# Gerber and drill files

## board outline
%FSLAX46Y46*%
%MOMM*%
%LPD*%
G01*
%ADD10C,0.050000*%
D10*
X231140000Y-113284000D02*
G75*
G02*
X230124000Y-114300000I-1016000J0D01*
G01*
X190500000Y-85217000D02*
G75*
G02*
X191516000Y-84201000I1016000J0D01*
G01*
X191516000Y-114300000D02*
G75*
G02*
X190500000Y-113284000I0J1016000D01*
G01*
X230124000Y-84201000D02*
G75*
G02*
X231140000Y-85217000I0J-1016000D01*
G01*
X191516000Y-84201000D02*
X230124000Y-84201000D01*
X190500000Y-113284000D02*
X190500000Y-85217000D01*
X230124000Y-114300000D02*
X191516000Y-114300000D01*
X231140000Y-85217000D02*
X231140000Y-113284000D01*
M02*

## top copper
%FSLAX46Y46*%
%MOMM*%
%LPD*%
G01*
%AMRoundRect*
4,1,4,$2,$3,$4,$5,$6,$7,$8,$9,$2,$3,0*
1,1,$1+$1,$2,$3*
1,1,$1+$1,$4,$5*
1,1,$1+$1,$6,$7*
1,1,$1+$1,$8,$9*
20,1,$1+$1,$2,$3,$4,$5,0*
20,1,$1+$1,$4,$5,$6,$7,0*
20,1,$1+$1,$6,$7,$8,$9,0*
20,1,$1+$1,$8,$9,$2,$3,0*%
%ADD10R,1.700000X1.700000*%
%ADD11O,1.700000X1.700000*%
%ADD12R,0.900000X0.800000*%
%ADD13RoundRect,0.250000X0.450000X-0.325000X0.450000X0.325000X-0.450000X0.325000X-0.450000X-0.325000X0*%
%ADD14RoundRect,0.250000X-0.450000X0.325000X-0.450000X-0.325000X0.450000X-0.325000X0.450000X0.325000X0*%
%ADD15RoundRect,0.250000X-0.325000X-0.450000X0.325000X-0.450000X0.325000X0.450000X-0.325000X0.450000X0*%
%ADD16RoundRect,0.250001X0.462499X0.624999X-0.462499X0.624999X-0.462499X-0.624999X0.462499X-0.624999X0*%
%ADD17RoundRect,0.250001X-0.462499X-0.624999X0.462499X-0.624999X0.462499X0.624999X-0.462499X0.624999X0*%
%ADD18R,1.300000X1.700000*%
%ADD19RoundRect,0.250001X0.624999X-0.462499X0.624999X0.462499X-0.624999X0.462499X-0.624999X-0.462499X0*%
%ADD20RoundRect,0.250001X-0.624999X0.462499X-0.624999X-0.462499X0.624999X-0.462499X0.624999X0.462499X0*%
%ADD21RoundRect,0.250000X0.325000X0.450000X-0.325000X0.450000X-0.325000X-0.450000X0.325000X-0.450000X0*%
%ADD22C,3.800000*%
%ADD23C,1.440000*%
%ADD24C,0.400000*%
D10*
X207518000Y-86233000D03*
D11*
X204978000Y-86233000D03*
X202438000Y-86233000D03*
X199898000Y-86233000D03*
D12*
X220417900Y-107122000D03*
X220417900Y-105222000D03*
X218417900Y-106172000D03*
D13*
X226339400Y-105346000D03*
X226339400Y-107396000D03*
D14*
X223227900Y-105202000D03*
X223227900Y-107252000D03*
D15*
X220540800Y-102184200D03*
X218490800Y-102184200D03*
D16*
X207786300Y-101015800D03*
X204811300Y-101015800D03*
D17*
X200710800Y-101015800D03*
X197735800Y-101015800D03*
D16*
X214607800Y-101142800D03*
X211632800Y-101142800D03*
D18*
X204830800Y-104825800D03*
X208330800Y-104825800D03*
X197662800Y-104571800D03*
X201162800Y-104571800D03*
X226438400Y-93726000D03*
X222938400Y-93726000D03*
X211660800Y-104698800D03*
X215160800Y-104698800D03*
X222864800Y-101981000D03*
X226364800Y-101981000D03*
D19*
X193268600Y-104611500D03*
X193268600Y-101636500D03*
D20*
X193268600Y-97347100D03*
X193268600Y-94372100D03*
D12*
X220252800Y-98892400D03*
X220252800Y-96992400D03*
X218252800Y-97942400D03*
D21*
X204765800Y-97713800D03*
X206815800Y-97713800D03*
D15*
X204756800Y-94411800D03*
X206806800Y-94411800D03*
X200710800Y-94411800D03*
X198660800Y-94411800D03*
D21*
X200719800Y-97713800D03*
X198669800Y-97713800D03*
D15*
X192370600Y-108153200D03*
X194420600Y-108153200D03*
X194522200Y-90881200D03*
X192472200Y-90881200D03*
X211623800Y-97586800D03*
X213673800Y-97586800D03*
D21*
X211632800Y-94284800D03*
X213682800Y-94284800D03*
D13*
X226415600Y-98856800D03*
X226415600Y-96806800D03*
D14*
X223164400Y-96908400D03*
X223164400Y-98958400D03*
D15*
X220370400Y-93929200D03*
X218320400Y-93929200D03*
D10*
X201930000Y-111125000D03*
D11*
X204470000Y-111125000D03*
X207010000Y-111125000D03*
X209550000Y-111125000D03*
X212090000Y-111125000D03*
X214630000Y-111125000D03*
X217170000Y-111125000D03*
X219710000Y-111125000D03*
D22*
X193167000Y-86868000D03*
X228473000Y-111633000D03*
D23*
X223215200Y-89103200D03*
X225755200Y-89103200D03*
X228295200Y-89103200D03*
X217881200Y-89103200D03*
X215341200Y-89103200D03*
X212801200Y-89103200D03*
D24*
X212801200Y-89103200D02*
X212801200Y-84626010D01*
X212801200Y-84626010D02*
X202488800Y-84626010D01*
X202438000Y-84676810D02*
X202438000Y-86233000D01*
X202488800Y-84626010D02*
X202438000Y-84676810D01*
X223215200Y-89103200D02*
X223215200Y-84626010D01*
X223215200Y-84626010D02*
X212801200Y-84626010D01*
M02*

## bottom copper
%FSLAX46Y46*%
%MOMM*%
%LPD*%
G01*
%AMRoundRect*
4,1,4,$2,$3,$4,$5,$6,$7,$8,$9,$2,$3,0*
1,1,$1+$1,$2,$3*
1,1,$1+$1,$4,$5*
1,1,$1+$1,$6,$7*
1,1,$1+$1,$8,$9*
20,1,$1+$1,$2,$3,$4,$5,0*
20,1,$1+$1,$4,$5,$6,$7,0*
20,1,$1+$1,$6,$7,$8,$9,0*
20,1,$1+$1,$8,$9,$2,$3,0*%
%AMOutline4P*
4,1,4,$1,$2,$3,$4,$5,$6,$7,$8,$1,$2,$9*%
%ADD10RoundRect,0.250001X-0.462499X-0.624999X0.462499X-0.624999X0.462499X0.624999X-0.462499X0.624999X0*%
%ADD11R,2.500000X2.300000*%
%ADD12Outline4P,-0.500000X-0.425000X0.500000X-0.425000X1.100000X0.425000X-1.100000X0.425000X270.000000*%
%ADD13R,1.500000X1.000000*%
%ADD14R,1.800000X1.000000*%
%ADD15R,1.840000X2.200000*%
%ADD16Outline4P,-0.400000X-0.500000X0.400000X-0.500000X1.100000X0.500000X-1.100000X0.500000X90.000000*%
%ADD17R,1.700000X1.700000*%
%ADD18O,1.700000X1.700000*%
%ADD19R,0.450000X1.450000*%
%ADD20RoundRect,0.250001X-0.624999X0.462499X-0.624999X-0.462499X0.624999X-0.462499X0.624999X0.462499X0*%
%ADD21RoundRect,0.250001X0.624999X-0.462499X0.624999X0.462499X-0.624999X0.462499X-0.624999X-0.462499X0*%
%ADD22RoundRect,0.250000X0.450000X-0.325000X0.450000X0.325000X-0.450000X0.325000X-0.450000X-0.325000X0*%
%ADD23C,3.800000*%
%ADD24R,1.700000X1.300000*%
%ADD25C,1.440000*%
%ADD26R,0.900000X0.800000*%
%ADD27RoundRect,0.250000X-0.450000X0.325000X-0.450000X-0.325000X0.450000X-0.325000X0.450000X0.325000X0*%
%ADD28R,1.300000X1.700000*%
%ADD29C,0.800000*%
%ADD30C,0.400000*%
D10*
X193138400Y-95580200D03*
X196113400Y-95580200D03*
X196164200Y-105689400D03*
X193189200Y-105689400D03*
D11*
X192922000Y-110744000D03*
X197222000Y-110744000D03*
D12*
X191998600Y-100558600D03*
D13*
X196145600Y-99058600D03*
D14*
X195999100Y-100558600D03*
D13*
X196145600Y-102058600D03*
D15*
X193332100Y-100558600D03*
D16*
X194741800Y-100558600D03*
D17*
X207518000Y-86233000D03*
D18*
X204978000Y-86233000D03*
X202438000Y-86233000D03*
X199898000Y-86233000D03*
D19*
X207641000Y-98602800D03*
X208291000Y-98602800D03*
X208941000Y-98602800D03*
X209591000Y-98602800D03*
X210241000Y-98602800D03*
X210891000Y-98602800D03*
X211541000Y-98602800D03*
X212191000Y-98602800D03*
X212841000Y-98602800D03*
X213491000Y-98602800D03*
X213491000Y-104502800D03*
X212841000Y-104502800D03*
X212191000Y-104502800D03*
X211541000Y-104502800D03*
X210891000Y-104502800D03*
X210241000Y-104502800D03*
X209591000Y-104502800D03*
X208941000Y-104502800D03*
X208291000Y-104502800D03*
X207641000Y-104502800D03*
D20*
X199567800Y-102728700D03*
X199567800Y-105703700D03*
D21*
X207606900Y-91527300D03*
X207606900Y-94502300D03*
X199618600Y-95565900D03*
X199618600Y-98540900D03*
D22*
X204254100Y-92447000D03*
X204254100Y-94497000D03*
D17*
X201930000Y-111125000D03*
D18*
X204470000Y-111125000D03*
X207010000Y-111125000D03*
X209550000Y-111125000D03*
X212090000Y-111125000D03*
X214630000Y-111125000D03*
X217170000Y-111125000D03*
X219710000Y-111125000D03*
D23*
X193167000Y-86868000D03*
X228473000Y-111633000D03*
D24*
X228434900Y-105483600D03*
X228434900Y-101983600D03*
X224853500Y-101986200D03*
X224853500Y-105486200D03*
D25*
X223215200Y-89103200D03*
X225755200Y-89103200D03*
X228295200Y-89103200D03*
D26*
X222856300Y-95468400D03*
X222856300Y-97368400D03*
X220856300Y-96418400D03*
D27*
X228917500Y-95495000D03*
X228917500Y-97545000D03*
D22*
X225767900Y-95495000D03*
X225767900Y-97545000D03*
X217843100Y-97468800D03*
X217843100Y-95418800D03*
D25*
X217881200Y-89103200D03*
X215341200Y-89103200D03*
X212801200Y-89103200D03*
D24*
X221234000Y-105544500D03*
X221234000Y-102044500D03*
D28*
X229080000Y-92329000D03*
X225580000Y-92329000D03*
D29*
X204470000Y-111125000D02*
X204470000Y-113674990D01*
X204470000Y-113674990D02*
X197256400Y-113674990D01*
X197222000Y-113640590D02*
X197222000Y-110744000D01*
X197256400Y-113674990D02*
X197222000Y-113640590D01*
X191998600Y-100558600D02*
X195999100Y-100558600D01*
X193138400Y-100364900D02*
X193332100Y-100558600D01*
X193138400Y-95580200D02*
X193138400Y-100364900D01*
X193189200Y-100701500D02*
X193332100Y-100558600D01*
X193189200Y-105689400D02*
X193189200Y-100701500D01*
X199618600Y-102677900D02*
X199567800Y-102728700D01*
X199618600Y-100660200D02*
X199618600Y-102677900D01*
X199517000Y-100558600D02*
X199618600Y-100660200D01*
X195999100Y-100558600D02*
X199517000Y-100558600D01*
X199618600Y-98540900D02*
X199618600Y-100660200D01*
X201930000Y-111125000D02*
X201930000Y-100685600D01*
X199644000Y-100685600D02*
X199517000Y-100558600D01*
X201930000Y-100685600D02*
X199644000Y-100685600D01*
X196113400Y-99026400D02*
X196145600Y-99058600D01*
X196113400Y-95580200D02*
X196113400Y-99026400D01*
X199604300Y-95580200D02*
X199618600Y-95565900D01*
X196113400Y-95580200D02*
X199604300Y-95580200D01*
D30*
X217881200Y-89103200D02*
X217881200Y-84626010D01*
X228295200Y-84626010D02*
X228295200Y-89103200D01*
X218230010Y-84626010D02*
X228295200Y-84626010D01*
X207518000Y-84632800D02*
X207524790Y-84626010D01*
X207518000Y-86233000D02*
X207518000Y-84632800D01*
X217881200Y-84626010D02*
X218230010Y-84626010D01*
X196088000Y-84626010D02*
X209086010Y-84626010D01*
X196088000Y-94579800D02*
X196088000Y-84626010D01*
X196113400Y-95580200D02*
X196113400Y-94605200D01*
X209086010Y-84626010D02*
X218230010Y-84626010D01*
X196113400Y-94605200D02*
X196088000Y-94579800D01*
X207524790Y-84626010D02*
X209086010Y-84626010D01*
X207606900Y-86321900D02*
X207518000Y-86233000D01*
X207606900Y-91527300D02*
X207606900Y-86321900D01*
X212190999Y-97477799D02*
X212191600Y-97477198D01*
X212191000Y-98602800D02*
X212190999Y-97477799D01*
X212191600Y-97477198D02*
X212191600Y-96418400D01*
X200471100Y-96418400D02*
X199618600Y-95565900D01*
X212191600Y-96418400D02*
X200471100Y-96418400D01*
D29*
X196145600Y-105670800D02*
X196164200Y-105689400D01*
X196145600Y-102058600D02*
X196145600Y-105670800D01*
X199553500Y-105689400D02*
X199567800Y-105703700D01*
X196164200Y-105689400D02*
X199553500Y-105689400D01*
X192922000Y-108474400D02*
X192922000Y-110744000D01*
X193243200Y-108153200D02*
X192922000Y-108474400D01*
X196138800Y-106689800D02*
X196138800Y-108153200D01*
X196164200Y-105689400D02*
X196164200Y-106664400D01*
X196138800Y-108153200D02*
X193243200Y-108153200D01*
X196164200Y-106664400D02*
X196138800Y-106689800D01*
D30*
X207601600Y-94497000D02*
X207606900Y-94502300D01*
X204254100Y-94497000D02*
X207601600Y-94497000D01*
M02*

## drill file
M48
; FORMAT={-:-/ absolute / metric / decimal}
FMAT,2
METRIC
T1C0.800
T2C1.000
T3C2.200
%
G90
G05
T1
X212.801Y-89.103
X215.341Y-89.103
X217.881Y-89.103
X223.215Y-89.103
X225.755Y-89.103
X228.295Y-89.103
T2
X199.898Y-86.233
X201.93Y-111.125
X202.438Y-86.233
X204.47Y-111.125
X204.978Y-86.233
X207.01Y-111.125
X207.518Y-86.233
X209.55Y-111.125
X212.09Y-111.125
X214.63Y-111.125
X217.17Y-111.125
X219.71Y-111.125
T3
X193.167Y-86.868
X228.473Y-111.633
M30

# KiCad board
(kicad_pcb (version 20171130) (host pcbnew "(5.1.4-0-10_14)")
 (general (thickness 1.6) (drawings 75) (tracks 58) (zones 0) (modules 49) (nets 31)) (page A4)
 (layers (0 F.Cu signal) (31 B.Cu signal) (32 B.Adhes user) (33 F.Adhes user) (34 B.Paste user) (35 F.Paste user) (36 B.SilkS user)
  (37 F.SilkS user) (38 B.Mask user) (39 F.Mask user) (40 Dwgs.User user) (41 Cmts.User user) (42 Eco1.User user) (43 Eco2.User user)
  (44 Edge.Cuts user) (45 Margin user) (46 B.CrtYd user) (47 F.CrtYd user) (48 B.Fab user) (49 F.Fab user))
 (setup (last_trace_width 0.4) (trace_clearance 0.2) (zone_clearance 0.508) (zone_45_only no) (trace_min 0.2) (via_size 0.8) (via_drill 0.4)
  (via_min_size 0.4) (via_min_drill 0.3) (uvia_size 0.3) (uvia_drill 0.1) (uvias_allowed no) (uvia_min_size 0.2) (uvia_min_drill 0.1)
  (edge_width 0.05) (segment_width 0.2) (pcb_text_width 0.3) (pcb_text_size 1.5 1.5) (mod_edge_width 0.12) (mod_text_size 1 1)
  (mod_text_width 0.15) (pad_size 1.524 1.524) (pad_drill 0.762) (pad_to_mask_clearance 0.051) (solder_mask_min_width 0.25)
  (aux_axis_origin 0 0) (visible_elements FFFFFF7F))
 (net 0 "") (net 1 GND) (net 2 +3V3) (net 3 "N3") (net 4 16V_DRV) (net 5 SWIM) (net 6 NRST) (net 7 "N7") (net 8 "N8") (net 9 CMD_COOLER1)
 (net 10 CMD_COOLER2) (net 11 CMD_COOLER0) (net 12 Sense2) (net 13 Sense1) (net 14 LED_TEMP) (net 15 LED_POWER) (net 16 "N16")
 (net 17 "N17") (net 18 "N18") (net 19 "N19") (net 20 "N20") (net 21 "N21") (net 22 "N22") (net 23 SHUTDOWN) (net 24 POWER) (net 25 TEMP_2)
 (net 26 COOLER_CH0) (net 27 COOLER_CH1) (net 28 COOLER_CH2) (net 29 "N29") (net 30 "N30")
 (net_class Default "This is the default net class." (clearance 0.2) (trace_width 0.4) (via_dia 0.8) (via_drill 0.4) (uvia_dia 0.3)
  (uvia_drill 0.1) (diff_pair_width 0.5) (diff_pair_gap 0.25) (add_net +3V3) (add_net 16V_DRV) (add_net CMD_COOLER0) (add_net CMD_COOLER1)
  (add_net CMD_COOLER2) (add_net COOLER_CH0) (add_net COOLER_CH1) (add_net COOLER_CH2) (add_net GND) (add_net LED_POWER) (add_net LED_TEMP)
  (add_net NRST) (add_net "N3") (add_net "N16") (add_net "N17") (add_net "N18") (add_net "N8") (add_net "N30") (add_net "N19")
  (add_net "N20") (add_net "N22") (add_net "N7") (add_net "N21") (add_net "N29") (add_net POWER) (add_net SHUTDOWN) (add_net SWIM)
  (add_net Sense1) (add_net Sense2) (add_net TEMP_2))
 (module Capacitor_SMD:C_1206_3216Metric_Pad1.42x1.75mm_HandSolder (layer B.Cu) (at 194.6259 95.5802)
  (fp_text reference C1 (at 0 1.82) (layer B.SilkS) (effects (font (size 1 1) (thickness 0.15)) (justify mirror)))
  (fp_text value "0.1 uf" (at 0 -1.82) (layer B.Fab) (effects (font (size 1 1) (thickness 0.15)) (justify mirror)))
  (pad 1 smd roundrect (at -1.4875 0) (size 1.425 1.75) (layers B.Cu B.Paste B.Mask) (roundrect_rratio 0.175439) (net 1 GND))
  (pad 2 smd roundrect (at 1.4875 0) (size 1.425 1.75) (layers B.Cu B.Paste B.Mask) (roundrect_rratio 0.175439) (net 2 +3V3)))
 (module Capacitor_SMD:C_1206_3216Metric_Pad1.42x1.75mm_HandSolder (layer B.Cu) (at 194.6767 105.6894)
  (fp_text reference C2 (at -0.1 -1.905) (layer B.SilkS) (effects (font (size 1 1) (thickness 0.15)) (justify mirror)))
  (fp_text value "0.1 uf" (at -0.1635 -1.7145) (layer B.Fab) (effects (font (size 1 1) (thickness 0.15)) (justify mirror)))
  (pad 2 smd roundrect (at 1.4875 0) (size 1.425 1.75) (layers B.Cu B.Paste B.Mask) (roundrect_rratio 0.175439) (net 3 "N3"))
  (pad 1 smd roundrect (at -1.4875 0) (size 1.425 1.75) (layers B.Cu B.Paste B.Mask) (roundrect_rratio 0.175439) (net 1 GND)))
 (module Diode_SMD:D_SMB (layer B.Cu) (at 195.072 110.744)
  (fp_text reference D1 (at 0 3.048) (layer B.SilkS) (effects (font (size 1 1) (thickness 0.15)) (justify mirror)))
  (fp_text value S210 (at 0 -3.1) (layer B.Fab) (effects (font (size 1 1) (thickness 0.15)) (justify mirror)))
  (pad 1 smd rect (at -2.15 0) (size 2.5 2.3) (layers B.Cu B.Paste B.Mask) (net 3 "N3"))
  (pad 2 smd rect (at 2.15 0) (size 2.5 2.3) (layers B.Cu B.Paste B.Mask) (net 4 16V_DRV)))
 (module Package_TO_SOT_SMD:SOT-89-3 (layer B.Cu) (at 194.6656 100.5586 180)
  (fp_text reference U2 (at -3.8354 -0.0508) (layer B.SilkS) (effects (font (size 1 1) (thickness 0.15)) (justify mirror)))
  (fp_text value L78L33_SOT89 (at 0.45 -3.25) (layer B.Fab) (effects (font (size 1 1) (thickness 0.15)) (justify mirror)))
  (pad 2 smd trapezoid (at 2.667 0 270) (size 1.6 0.85) (rect_delta 0 -0.6) (layers B.Cu B.Paste B.Mask) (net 1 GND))
  (pad 1 smd rect (at -1.48 1.5 270) (size 1 1.5) (layers B.Cu B.Paste B.Mask) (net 2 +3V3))
  (pad 2 smd rect (at -1.3335 0 270) (size 1 1.8) (layers B.Cu B.Paste B.Mask) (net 1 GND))
  (pad 3 smd rect (at -1.48 -1.5 270) (size 1 1.5) (layers B.Cu B.Paste B.Mask) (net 3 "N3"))
  (pad 2 smd rect (at 1.3335 0 270) (size 2.2 1.84) (layers B.Cu B.Paste B.Mask) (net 1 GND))
  (pad 2 smd trapezoid (at -0.0762 0 90) (size 1.5 1) (rect_delta 0 -0.7) (layers B.Cu B.Paste B.Mask) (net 1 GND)))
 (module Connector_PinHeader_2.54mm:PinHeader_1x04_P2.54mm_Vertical (layer B.Cu) (at 207.518 86.233 90)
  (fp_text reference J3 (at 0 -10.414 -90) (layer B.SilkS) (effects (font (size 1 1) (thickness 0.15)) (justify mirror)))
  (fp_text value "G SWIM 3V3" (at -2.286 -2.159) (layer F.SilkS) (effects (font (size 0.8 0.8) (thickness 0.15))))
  (pad 1 thru_hole rect (at 0 0 90) (size 1.7 1.7) (drill 1) (layers *.Cu *.Mask) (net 2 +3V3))
  (pad 2 thru_hole oval (at 0 -2.54 90) (size 1.7 1.7) (drill 1) (layers *.Cu *.Mask) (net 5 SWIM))
  (pad 3 thru_hole oval (at 0 -5.08 90) (size 1.7 1.7) (drill 1) (layers *.Cu *.Mask) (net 1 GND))
  (pad 4 thru_hole oval (at 0 -7.62 90) (size 1.7 1.7) (drill 1) (layers *.Cu *.Mask) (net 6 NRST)))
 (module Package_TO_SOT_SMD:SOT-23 (layer F.Cu) (at 219.4179 106.172 180)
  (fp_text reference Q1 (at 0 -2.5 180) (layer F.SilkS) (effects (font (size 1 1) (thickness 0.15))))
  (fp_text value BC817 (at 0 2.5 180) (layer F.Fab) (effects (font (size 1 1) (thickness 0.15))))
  (pad 1 smd rect (at -1 -0.95 180) (size 0.9 0.8) (layers F.Cu F.Paste F.Mask) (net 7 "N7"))
  (pad 2 smd rect (at -1 0.95 180) (size 0.9 0.8) (layers F.Cu F.Paste F.Mask) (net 1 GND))
  (pad 3 smd rect (at 1 0 180) (size 0.9 0.8) (layers F.Cu F.Paste F.Mask) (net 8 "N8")))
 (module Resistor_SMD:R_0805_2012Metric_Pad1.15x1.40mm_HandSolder (layer F.Cu) (at 226.3394 106.371 90)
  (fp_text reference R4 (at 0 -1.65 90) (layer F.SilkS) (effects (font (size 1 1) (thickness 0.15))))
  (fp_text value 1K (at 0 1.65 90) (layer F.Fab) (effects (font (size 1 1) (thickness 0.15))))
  (pad 2 smd roundrect (at 1.025 0 90) (size 1.15 1.4) (layers F.Cu F.Paste F.Mask) (roundrect_rratio 0.217391) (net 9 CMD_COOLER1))
  (pad 1 smd roundrect (at -1.025 0 90) (size 1.15 1.4) (layers F.Cu F.Paste F.Mask) (roundrect_rratio 0.217391) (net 7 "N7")))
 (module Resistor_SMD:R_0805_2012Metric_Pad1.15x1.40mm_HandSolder (layer F.Cu) (at 223.2279 106.227 270)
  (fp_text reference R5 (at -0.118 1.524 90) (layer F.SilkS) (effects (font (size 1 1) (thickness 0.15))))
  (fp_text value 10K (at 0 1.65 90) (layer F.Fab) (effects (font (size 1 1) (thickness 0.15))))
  (pad 1 smd roundrect (at -1.025 0 270) (size 1.15 1.4) (layers F.Cu F.Paste F.Mask) (roundrect_rratio 0.217391) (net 1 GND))
  (pad 2 smd roundrect (at 1.025 0 270) (size 1.15 1.4) (layers F.Cu F.Paste F.Mask) (roundrect_rratio 0.217391) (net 7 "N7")))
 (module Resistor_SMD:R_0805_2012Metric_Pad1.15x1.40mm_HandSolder (layer F.Cu) (at 219.5158 102.1842)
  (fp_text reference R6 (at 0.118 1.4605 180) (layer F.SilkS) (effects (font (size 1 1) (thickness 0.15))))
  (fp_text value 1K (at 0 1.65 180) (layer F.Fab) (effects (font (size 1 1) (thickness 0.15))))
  (pad 2 smd roundrect (at 1.025 0) (size 1.15 1.4) (layers F.Cu F.Paste F.Mask) (roundrect_rratio 0.217391) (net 4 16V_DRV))
  (pad 1 smd roundrect (at -1.025 0) (size 1.15 1.4) (layers F.Cu F.Paste F.Mask) (roundrect_rratio 0.217391) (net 8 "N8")))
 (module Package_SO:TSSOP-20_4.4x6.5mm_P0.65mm (layer B.Cu) (at 210.566 101.5528 270)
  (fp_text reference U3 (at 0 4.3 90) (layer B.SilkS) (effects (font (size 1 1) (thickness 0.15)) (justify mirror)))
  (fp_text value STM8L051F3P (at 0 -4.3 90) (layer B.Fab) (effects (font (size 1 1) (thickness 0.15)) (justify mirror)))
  (pad 1 smd rect (at -2.95 2.925 270) (size 1.45 0.45) (layers B.Cu B.Paste B.Mask) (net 9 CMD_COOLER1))
  (pad 2 smd rect (at -2.95 2.275 270) (size 1.45 0.45) (layers B.Cu B.Paste B.Mask) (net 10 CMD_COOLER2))
  (pad 3 smd rect (at -2.95 1.625 270) (size 1.45 0.45) (layers B.Cu B.Paste B.Mask) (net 5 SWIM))
  (pad 4 smd rect (at -2.95 0.975 270) (size 1.45 0.45) (layers B.Cu B.Paste B.Mask) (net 6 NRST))
  (pad 5 smd rect (at -2.95 0.325 270) (size 1.45 0.45) (layers B.Cu B.Paste B.Mask) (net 1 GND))
  (pad 6 smd rect (at -2.95 -0.325 270) (size 1.45 0.45) (layers B.Cu B.Paste B.Mask) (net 1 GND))
  (pad 7 smd rect (at -2.95 -0.975 270) (size 1.45 0.45) (layers B.Cu B.Paste B.Mask) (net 1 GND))
  (pad 8 smd rect (at -2.95 -1.625 270) (size 1.45 0.45) (layers B.Cu B.Paste B.Mask) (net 2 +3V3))
  (pad 9 smd rect (at -2.95 -2.275 270) (size 1.45 0.45) (layers B.Cu B.Paste B.Mask) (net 1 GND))
  (pad 10 smd rect (at -2.95 -2.925 270) (size 1.45 0.45) (layers B.Cu B.Paste B.Mask) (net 1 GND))
  (pad 11 smd rect (at 2.95 -2.925 270) (size 1.45 0.45) (layers B.Cu B.Paste B.Mask) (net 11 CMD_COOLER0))
  (pad 12 smd rect (at 2.95 -2.275 270) (size 1.45 0.45) (layers B.Cu B.Paste B.Mask) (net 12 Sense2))
  (pad 13 smd rect (at 2.95 -1.625 270) (size 1.45 0.45) (layers B.Cu B.Paste B.Mask) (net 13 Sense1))
  (pad 14 smd rect (at 2.95 -0.975 270) (size 1.45 0.45) (layers B.Cu B.Paste B.Mask) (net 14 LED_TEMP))
  (pad 15 smd rect (at 2.95 -0.325 270) (size 1.45 0.45) (layers B.Cu B.Paste B.Mask) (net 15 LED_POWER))
  (pad 16 smd rect (at 2.95 0.325 270) (size 1.45 0.45) (layers B.Cu B.Paste B.Mask) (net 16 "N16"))
  (pad 17 smd rect (at 2.95 0.975 270) (size 1.45 0.45) (layers B.Cu B.Paste B.Mask) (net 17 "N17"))
  (pad 18 smd rect (at 2.95 1.625 270) (size 1.45 0.45) (layers B.Cu B.Paste B.Mask))
  (pad 19 smd rect (at 2.95 2.275 270) (size 1.45 0.45) (layers B.Cu B.Paste B.Mask))
  (pad 20 smd rect (at 2.95 2.925 270) (size 1.45 0.45) (layers B.Cu B.Paste B.Mask) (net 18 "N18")))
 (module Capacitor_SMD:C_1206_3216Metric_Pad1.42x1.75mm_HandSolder (layer B.Cu) (at 199.5678 104.2162 270)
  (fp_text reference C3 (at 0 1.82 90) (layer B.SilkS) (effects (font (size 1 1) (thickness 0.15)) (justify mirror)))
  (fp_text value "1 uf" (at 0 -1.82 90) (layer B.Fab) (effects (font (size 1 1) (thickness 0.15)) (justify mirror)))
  (pad 1 smd roundrect (at -1.4875 0 270) (size 1.425 1.75) (layers B.Cu B.Paste B.Mask) (roundrect_rratio 0.175439) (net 1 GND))
  (pad 2 smd roundrect (at 1.4875 0 270) (size 1.425 1.75) (layers B.Cu B.Paste B.Mask) (roundrect_rratio 0.175439) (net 3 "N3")))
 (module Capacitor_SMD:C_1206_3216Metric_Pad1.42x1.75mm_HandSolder (layer B.Cu) (at 207.6069 93.0148 90)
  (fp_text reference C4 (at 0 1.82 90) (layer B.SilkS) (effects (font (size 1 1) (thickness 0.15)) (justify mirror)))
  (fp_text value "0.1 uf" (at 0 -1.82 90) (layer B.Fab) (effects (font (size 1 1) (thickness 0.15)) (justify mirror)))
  (pad 2 smd roundrect (at 1.4875 0 90) (size 1.425 1.75) (layers B.Cu B.Paste B.Mask) (roundrect_rratio 0.175439) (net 2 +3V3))
  (pad 1 smd roundrect (at -1.4875 0 90) (size 1.425 1.75) (layers B.Cu B.Paste B.Mask) (roundrect_rratio 0.175439) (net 6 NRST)))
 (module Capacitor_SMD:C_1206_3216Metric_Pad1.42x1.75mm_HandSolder (layer F.Cu) (at 206.2988 101.0158 180)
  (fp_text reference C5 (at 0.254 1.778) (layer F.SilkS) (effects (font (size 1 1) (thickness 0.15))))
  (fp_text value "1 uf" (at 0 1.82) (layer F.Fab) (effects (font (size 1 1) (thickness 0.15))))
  (pad 1 smd roundrect (at -1.4875 0 180) (size 1.425 1.75) (layers F.Cu F.Paste F.Mask) (roundrect_rratio 0.175439) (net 1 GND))
  (pad 2 smd roundrect (at 1.4875 0 180) (size 1.425 1.75) (layers F.Cu F.Paste F.Mask) (roundrect_rratio 0.175439) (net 16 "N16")))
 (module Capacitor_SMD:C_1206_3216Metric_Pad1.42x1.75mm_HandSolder (layer B.Cu) (at 199.6186 97.0534 90)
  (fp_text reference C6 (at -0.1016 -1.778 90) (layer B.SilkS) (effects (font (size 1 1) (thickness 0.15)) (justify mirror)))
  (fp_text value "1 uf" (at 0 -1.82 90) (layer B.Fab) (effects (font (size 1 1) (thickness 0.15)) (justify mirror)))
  (pad 2 smd roundrect (at 1.4875 0 90) (size 1.425 1.75) (layers B.Cu B.Paste B.Mask) (roundrect_rratio 0.175439) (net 2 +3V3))
  (pad 1 smd roundrect (at -1.4875 0 90) (size 1.425 1.75) (layers B.Cu B.Paste B.Mask) (roundrect_rratio 0.175439) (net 1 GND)))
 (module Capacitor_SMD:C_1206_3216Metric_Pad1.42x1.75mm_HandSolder (layer F.Cu) (at 199.2233 101.0158)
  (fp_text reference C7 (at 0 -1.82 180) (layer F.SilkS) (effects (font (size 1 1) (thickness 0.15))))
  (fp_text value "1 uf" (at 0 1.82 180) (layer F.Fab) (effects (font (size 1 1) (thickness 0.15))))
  (pad 2 smd roundrect (at 1.4875 0) (size 1.425 1.75) (layers F.Cu F.Paste F.Mask) (roundrect_rratio 0.175439) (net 17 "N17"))
  (pad 1 smd roundrect (at -1.4875 0) (size 1.425 1.75) (layers F.Cu F.Paste F.Mask) (roundrect_rratio 0.175439) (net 1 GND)))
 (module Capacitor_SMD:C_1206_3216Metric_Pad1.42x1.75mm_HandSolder (layer F.Cu) (at 213.1203 101.1428 180)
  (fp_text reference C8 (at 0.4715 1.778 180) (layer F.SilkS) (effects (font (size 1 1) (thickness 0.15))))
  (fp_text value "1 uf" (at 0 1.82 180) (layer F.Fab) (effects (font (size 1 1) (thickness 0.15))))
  (pad 1 smd roundrect (at -1.4875 0 180) (size 1.425 1.75) (layers F.Cu F.Paste F.Mask) (roundrect_rratio 0.175439) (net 1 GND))
  (pad 2 smd roundrect (at 1.4875 0 180) (size 1.425 1.75) (layers F.Cu F.Paste F.Mask) (roundrect_rratio 0.175439) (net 18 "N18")))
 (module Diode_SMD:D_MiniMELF (layer F.Cu) (at 206.5808 104.8258)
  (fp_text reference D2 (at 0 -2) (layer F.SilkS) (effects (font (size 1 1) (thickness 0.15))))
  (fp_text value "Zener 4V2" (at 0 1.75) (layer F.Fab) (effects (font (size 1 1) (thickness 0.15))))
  (pad 1 smd rect (at -1.75 0) (size 1.3 1.7) (layers F.Cu F.Paste F.Mask) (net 16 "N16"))
  (pad 2 smd rect (at 1.75 0) (size 1.3 1.7) (layers F.Cu F.Paste F.Mask) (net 1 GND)))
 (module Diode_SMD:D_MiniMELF (layer F.Cu) (at 199.4128 104.5718 180)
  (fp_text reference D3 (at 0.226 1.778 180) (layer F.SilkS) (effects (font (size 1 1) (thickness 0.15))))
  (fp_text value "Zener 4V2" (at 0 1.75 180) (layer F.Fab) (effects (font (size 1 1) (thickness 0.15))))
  (pad 2 smd rect (at 1.75 0 180) (size 1.3 1.7) (layers F.Cu F.Paste F.Mask) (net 1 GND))
  (pad 1 smd rect (at -1.75 0 180) (size 1.3 1.7) (layers F.Cu F.Paste F.Mask) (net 17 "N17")))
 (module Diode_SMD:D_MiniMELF (layer F.Cu) (at 224.6884 93.726 180)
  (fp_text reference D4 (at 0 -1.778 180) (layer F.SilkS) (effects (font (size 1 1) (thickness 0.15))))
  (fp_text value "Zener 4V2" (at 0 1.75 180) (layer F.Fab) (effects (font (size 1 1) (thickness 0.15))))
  (pad 1 smd rect (at -1.75 0 180) (size 1.3 1.7) (layers F.Cu F.Paste F.Mask) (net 10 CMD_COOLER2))
  (pad 2 smd rect (at 1.75 0 180) (size 1.3 1.7) (layers F.Cu F.Paste F.Mask) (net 1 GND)))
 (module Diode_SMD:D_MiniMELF (layer F.Cu) (at 213.4108 104.6988)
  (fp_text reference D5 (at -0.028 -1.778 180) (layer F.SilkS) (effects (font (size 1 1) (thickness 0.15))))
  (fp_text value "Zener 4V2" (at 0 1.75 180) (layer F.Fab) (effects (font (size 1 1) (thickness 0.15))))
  (pad 1 smd rect (at -1.75 0) (size 1.3 1.7) (layers F.Cu F.Paste F.Mask) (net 18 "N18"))
  (pad 2 smd rect (at 1.75 0) (size 1.3 1.7) (layers F.Cu F.Paste F.Mask) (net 1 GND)))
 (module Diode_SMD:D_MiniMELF (layer F.Cu) (at 224.6148 101.981 180)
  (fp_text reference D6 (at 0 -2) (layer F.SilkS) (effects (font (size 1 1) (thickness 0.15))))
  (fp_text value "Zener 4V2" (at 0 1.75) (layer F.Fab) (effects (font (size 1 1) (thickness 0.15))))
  (pad 2 smd rect (at 1.75 0 180) (size 1.3 1.7) (layers F.Cu F.Paste F.Mask) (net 1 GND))
  (pad 1 smd rect (at -1.75 0 180) (size 1.3 1.7) (layers F.Cu F.Paste F.Mask) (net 9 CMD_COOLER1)))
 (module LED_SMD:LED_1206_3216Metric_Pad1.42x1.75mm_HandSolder (layer F.Cu) (at 193.2686 103.124 90)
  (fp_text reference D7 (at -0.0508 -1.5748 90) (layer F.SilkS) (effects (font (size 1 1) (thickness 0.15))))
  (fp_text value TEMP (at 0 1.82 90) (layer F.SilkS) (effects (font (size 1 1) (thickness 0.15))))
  (pad 1 smd roundrect (at -1.4875 0 90) (size 1.425 1.75) (layers F.Cu F.Paste F.Mask) (roundrect_rratio 0.175439) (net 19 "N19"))
  (pad 2 smd roundrect (at 1.4875 0 90) (size 1.425 1.75) (layers F.Cu F.Paste F.Mask) (roundrect_rratio 0.175439) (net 14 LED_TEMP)))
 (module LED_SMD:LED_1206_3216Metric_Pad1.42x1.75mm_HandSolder (layer F.Cu) (at 193.2686 95.8596 270)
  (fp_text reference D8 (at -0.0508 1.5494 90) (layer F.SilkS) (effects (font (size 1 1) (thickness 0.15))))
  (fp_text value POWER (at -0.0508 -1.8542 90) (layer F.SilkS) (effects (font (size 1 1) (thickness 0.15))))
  (pad 2 smd roundrect (at 1.4875 0 270) (size 1.425 1.75) (layers F.Cu F.Paste F.Mask) (roundrect_rratio 0.175439) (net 15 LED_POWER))
  (pad 1 smd roundrect (at -1.4875 0 270) (size 1.425 1.75) (layers F.Cu F.Paste F.Mask) (roundrect_rratio 0.175439) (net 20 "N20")))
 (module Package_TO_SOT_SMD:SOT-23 (layer F.Cu) (at 219.2528 97.9424 180)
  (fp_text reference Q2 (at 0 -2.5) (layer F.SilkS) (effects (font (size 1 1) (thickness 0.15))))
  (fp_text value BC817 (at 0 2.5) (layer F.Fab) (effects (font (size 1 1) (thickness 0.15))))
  (pad 1 smd rect (at -1 -0.95 180) (size 0.9 0.8) (layers F.Cu F.Paste F.Mask) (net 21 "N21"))
  (pad 2 smd rect (at -1 0.95 180) (size 0.9 0.8) (layers F.Cu F.Paste F.Mask) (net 1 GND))
  (pad 3 smd rect (at 1 0 180) (size 0.9 0.8) (layers F.Cu F.Paste F.Mask) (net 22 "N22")))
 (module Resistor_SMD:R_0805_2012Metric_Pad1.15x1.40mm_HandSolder (layer F.Cu) (at 205.7908 97.7138 180)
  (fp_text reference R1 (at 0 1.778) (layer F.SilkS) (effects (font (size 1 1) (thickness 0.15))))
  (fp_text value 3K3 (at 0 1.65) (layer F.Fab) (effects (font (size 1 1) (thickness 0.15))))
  (pad 2 smd roundrect (at 1.025 0 180) (size 1.15 1.4) (layers F.Cu F.Paste F.Mask) (roundrect_rratio 0.217391) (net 16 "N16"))
  (pad 1 smd roundrect (at -1.025 0 180) (size 1.15 1.4) (layers F.Cu F.Paste F.Mask) (roundrect_rratio 0.217391) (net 1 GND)))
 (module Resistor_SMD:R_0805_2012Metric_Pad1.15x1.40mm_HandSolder (layer B.Cu) (at 204.2541 93.472 90)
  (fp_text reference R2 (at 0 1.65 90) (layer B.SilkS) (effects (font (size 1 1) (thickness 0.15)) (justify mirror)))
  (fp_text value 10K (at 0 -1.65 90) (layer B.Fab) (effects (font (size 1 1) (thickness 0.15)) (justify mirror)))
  (pad 2 smd roundrect (at 1.025 0 90) (size 1.15 1.4) (layers B.Cu B.Paste B.Mask) (roundrect_rratio 0.217391) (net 1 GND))
  (pad 1 smd roundrect (at -1.025 0 90) (size 1.15 1.4) (layers B.Cu B.Paste B.Mask) (roundrect_rratio 0.217391) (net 6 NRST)))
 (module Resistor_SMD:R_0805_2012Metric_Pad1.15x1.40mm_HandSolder (layer F.Cu) (at 205.7818 94.4118)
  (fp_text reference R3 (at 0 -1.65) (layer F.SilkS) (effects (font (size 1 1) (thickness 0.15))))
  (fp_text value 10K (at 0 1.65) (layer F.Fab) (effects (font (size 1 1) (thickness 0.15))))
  (pad 1 smd roundrect (at -1.025 0) (size 1.15 1.4) (layers F.Cu F.Paste F.Mask) (roundrect_rratio 0.217391) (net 16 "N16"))
  (pad 2 smd roundrect (at 1.025 0) (size 1.15 1.4) (layers F.Cu F.Paste F.Mask) (roundrect_rratio 0.217391) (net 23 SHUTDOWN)))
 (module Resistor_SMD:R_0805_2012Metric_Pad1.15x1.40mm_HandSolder (layer F.Cu) (at 199.6858 94.4118)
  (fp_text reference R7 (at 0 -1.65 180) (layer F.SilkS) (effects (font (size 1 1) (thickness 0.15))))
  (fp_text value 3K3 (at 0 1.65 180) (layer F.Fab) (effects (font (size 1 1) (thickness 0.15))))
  (pad 2 smd roundrect (at 1.025 0) (size 1.15 1.4) (layers F.Cu F.Paste F.Mask) (roundrect_rratio 0.217391) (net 17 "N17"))
  (pad 1 smd roundrect (at -1.025 0) (size 1.15 1.4) (layers F.Cu F.Paste F.Mask) (roundrect_rratio 0.217391) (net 1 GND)))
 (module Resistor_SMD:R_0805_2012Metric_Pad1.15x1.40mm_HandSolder (layer F.Cu) (at 199.6948 97.7138 180)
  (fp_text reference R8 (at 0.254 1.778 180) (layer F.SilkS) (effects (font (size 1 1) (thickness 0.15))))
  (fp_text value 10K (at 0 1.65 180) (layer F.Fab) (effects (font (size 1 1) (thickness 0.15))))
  (pad 1 smd roundrect (at -1.025 0 180) (size 1.15 1.4) (layers F.Cu F.Paste F.Mask) (roundrect_rratio 0.217391) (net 17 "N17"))
  (pad 2 smd roundrect (at 1.025 0 180) (size 1.15 1.4) (layers F.Cu F.Paste F.Mask) (roundrect_rratio 0.217391) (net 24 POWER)))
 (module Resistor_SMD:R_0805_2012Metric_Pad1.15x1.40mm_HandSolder (layer F.Cu) (at 193.3956 108.1532)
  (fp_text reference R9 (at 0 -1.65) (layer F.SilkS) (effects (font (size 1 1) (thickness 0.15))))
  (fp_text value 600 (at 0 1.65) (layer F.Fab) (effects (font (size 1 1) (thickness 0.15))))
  (pad 1 smd roundrect (at -1.025 0) (size 1.15 1.4) (layers F.Cu F.Paste F.Mask) (roundrect_rratio 0.217391) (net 1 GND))
  (pad 2 smd roundrect (at 1.025 0) (size 1.15 1.4) (layers F.Cu F.Paste F.Mask) (roundrect_rratio 0.217391) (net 19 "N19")))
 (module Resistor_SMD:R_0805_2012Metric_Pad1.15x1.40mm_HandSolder (layer F.Cu) (at 193.4972 90.8812)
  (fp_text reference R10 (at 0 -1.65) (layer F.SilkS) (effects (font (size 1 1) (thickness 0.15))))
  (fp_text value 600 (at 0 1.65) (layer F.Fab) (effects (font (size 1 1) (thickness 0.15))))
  (pad 2 smd roundrect (at 1.025 0) (size 1.15 1.4) (layers F.Cu F.Paste F.Mask) (roundrect_rratio 0.217391) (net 20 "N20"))
  (pad 1 smd roundrect (at -1.025 0) (size 1.15 1.4) (layers F.Cu F.Paste F.Mask) (roundrect_rratio 0.217391) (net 1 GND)))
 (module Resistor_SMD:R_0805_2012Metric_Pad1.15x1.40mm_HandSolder (layer F.Cu) (at 212.6488 97.5868)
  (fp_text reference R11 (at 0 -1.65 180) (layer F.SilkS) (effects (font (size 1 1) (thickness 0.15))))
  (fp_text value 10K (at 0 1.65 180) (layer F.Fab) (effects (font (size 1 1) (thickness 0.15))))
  (pad 1 smd roundrect (at -1.025 0) (size 1.15 1.4) (layers F.Cu F.Paste F.Mask) (roundrect_rratio 0.217391) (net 18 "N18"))
  (pad 2 smd roundrect (at 1.025 0) (size 1.15 1.4) (layers F.Cu F.Paste F.Mask) (roundrect_rratio 0.217391) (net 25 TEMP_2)))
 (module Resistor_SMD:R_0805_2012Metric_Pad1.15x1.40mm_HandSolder (layer F.Cu) (at 212.6578 94.2848 180)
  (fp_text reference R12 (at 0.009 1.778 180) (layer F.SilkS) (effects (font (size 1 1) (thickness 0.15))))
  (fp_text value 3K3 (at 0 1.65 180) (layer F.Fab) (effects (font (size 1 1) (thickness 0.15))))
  (pad 2 smd roundrect (at 1.025 0 180) (size 1.15 1.4) (layers F.Cu F.Paste F.Mask) (roundrect_rratio 0.217391) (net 18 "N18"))
  (pad 1 smd roundrect (at -1.025 0 180) (size 1.15 1.4) (layers F.Cu F.Paste F.Mask) (roundrect_rratio 0.217391) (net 1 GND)))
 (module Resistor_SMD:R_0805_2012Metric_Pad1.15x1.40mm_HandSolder (layer F.Cu) (at 226.4156 97.8318 90)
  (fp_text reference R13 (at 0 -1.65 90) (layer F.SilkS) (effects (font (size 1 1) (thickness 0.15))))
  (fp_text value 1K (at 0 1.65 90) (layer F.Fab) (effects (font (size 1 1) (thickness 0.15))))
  (pad 1 smd roundrect (at -1.025 0 90) (size 1.15 1.4) (layers F.Cu F.Paste F.Mask) (roundrect_rratio 0.217391) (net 21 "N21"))
  (pad 2 smd roundrect (at 1.025 0 90) (size 1.15 1.4) (layers F.Cu F.Paste F.Mask) (roundrect_rratio 0.217391) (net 10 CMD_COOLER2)))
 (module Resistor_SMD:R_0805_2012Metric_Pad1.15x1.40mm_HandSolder (layer F.Cu) (at 223.1644 97.9334 270)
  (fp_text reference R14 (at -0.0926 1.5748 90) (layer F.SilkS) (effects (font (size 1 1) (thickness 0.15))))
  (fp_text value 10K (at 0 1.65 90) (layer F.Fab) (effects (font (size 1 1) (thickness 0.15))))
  (pad 1 smd roundrect (at -1.025 0 270) (size 1.15 1.4) (layers F.Cu F.Paste F.Mask) (roundrect_rratio 0.217391) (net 1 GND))
  (pad 2 smd roundrect (at 1.025 0 270) (size 1.15 1.4) (layers F.Cu F.Paste F.Mask) (roundrect_rratio 0.217391) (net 21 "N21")))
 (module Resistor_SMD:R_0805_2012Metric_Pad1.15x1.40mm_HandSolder (layer F.Cu) (at 219.3454 93.9292)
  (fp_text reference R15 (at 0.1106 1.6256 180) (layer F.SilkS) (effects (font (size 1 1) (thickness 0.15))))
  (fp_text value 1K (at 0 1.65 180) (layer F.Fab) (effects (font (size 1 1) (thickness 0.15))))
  (pad 2 smd roundrect (at 1.025 0) (size 1.15 1.4) (layers F.Cu F.Paste F.Mask) (roundrect_rratio 0.217391) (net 4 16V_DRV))
  (pad 1 smd roundrect (at -1.025 0) (size 1.15 1.4) (layers F.Cu F.Paste F.Mask) (roundrect_rratio 0.217391) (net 22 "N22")))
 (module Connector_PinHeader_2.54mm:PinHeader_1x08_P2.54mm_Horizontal (layer B.Cu) (at 201.93 111.125 270)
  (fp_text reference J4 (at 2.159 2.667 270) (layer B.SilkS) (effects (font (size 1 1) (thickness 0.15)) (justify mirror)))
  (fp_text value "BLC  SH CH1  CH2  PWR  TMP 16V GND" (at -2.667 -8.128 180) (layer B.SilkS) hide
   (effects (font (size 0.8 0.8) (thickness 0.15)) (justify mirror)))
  (pad 1 thru_hole rect (at 0 0 270) (size 1.7 1.7) (drill 1) (layers *.Cu *.Mask) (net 1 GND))
  (pad 2 thru_hole oval (at 0 -2.54 270) (size 1.7 1.7) (drill 1) (layers *.Cu *.Mask) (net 4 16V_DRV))
  (pad 3 thru_hole oval (at 0 -5.08 270) (size 1.7 1.7) (drill 1) (layers *.Cu *.Mask) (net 25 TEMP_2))
  (pad 4 thru_hole oval (at 0 -7.62 270) (size 1.7 1.7) (drill 1) (layers *.Cu *.Mask) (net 24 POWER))
  (pad 5 thru_hole oval (at 0 -10.16 270) (size 1.7 1.7) (drill 1) (layers *.Cu *.Mask) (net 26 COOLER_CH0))
  (pad 6 thru_hole oval (at 0 -12.7 270) (size 1.7 1.7) (drill 1) (layers *.Cu *.Mask) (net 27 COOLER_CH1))
  (pad 7 thru_hole oval (at 0 -15.24 270) (size 1.7 1.7) (drill 1) (layers *.Cu *.Mask) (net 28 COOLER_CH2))
  (pad 8 thru_hole oval (at 0 -17.78 270) (size 1.7 1.7) (drill 1) (layers *.Cu *.Mask) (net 23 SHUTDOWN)))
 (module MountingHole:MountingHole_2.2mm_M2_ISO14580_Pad (layer F.Cu) (at 193.167 86.868)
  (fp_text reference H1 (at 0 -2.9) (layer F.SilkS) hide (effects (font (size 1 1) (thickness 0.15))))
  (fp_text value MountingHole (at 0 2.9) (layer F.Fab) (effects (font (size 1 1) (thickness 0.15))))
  (pad 1 thru_hole circle (at 0 0) (size 3.8 3.8) (drill 2.2) (layers *.Cu *.Mask)))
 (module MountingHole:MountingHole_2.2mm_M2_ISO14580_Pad (layer F.Cu) (at 228.473 111.633)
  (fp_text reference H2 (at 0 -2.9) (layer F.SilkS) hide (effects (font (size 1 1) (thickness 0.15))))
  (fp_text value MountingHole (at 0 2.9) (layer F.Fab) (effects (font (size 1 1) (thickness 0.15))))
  (pad 1 thru_hole circle (at 0 0) (size 3.8 3.8) (drill 2.2) (layers *.Cu *.Mask)))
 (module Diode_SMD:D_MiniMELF (layer B.Cu) (at 228.4349 103.7336 90)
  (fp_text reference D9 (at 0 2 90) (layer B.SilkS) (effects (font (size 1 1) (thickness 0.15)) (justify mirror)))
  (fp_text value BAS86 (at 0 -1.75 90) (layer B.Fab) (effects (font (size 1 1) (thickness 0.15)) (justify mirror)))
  (pad 1 smd rect (at -1.75 0 90) (size 1.3 1.7) (layers B.Cu B.Paste B.Mask) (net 28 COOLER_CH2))
  (pad 2 smd rect (at 1.75 0 90) (size 1.3 1.7) (layers B.Cu B.Paste B.Mask) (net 22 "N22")))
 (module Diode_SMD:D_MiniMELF (layer B.Cu) (at 224.8535 103.7362 90)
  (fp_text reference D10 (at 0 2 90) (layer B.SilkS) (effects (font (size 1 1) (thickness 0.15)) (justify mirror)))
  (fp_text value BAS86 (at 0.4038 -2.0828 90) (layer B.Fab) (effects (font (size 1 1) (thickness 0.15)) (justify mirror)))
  (pad 2 smd rect (at 1.75 0 90) (size 1.3 1.7) (layers B.Cu B.Paste B.Mask) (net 8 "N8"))
  (pad 1 smd rect (at -1.75 0 90) (size 1.3 1.7) (layers B.Cu B.Paste B.Mask) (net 27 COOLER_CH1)))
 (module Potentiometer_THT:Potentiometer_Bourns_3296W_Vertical (layer F.Cu) (at 228.2952 89.1032)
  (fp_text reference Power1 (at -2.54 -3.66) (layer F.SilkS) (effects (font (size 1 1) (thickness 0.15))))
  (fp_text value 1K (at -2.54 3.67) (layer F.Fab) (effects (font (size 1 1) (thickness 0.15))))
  (pad 3 thru_hole circle (at -5.08 0) (size 1.44 1.44) (drill 0.8) (layers *.Cu *.Mask) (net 1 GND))
  (pad 2 thru_hole circle (at -2.54 0) (size 1.44 1.44) (drill 0.8) (layers *.Cu *.Mask) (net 13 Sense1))
  (pad 1 thru_hole circle (at 0 0) (size 1.44 1.44) (drill 0.8) (layers *.Cu *.Mask) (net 2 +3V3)))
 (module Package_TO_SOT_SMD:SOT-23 (layer B.Cu) (at 221.8563 96.4184 180)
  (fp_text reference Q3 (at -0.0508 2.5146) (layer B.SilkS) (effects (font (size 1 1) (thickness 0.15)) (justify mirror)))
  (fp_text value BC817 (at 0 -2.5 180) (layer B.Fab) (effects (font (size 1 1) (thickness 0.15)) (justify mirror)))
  (pad 1 smd rect (at -1 0.95 180) (size 0.9 0.8) (layers B.Cu B.Paste B.Mask) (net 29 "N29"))
  (pad 2 smd rect (at -1 -0.95 180) (size 0.9 0.8) (layers B.Cu B.Paste B.Mask) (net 1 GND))
  (pad 3 smd rect (at 1 0 180) (size 0.9 0.8) (layers B.Cu B.Paste B.Mask) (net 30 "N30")))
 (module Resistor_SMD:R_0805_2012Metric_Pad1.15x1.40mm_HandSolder (layer B.Cu) (at 228.9175 96.52 270)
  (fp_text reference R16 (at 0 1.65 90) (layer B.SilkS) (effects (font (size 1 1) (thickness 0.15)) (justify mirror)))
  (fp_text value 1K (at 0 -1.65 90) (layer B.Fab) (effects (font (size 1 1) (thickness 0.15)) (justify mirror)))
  (pad 1 smd roundrect (at -1.025 0 270) (size 1.15 1.4) (layers B.Cu B.Paste B.Mask) (roundrect_rratio 0.217391) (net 29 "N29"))
  (pad 2 smd roundrect (at 1.025 0 270) (size 1.15 1.4) (layers B.Cu B.Paste B.Mask) (roundrect_rratio 0.217391) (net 11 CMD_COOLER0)))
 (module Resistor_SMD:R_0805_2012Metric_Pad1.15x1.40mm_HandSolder (layer B.Cu) (at 225.7679 96.52 90)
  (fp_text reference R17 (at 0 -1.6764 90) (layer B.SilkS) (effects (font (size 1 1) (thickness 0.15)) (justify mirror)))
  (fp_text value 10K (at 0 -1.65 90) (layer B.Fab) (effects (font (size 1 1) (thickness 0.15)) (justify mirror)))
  (pad 2 smd roundrect (at 1.025 0 90) (size 1.15 1.4) (layers B.Cu B.Paste B.Mask) (roundrect_rratio 0.217391) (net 29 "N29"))
  (pad 1 smd roundrect (at -1.025 0 90) (size 1.15 1.4) (layers B.Cu B.Paste B.Mask) (roundrect_rratio 0.217391) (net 1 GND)))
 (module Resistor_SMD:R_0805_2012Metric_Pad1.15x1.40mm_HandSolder (layer B.Cu) (at 217.8431 96.4438 90)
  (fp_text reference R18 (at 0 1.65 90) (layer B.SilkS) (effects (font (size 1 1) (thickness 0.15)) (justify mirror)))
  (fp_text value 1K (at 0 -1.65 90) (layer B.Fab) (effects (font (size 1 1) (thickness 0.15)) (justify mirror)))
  (pad 1 smd roundrect (at -1.025 0 90) (size 1.15 1.4) (layers B.Cu B.Paste B.Mask) (roundrect_rratio 0.217391) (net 30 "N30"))
  (pad 2 smd roundrect (at 1.025 0 90) (size 1.15 1.4) (layers B.Cu B.Paste B.Mask) (roundrect_rratio 0.217391) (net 4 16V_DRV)))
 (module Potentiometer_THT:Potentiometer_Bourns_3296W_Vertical (layer F.Cu) (at 217.8812 89.1032)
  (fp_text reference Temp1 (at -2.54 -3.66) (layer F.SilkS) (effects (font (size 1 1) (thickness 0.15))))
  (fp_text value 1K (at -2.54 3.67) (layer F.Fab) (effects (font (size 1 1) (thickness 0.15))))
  (pad 1 thru_hole circle (at 0 0) (size 1.44 1.44) (drill 0.8) (layers *.Cu *.Mask) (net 2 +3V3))
  (pad 2 thru_hole circle (at -2.54 0) (size 1.44 1.44) (drill 0.8) (layers *.Cu *.Mask) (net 12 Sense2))
  (pad 3 thru_hole circle (at -5.08 0) (size 1.44 1.44) (drill 0.8) (layers *.Cu *.Mask) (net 1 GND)))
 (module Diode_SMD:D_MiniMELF (layer B.Cu) (at 221.234 103.7945 90)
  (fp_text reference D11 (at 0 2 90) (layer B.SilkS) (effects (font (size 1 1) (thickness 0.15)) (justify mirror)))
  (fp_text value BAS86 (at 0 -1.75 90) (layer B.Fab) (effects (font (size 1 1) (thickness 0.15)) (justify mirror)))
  (pad 1 smd rect (at -1.75 0 90) (size 1.3 1.7) (layers B.Cu B.Paste B.Mask) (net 26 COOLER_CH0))
  (pad 2 smd rect (at 1.75 0 90) (size 1.3 1.7) (layers B.Cu B.Paste B.Mask) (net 30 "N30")))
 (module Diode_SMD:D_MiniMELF (layer B.Cu) (at 227.33 92.329 180)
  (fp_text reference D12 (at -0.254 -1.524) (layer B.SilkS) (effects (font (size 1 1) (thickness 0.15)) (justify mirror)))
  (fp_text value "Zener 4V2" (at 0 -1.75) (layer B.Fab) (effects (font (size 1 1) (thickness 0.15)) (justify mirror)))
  (pad 1 smd rect (at -1.75 0 180) (size 1.3 1.7) (layers B.Cu B.Paste B.Mask) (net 11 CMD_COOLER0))
  (pad 2 smd rect (at 1.75 0 180) (size 1.3 1.7) (layers B.Cu B.Paste B.Mask) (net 1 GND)))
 (gr_arc (start 230.124 113.284) (end 230.124 114.3) (angle -90) (layer Edge.Cuts) (width 0.05))
 (gr_arc (start 191.516 85.217) (end 191.516 84.201) (angle -90) (layer Edge.Cuts) (width 0.05))
 (gr_arc (start 191.516 113.284) (end 190.5 113.284) (angle -90) (layer Edge.Cuts) (width 0.05))
 (gr_arc (start 230.124 85.217) (end 231.14 85.217) (angle -90) (layer Edge.Cuts) (width 0.05))
 (gr_line (start 191.516 84.201) (end 230.124 84.201) (layer Edge.Cuts) (width 0.05))
 (gr_line (start 190.5 113.284) (end 190.5 85.217) (layer Edge.Cuts) (width 0.05))
 (gr_line (start 230.124 114.3) (end 191.516 114.3) (layer Edge.Cuts) (width 0.05))
 (gr_line (start 231.14 85.217) (end 231.14 113.284) (layer Edge.Cuts) (width 0.05))
 (segment (start 204.47 111.125) (end 204.47 113.67499) (width 0.8) (layer B.Cu) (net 4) (status 10))
 (segment (start 204.47 113.67499) (end 197.2564 113.67499) (width 0.8) (layer B.Cu) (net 4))
 (segment (start 197.222 113.64059) (end 197.222 110.744) (width 0.8) (layer B.Cu) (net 4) (status 20))
 (segment (start 197.2564 113.67499) (end 197.222 113.64059) (width 0.8) (layer B.Cu) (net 4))
 (segment (start 191.9986 100.5586) (end 195.9991 100.5586) (width 0.8) (layer B.Cu) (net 1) (status 30))
 (segment (start 193.1384 100.3649) (end 193.3321 100.5586) (width 0.8) (layer B.Cu) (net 1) (status 30))
 (segment (start 193.1384 95.5802) (end 193.1384 100.3649) (width 0.8) (layer B.Cu) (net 1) (status 30))
 (segment (start 193.1892 100.7015) (end 193.3321 100.5586) (width 0.8) (layer B.Cu) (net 1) (status 30))
 (segment (start 193.1892 105.6894) (end 193.1892 100.7015) (width 0.8) (layer B.Cu) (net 1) (status 30))
 (segment (start 199.6186 102.6779) (end 199.5678 102.7287) (width 0.8) (layer B.Cu) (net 1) (status 30))
 (segment (start 199.6186 100.6602) (end 199.6186 102.6779) (width 0.8) (layer B.Cu) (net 1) (status 20))
 (segment (start 199.517 100.5586) (end 199.6186 100.6602) (width 0.8) (layer B.Cu) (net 1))
 (segment (start 195.9991 100.5586) (end 199.517 100.5586) (width 0.8) (layer B.Cu) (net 1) (status 10))
 (segment (start 199.6186 98.5409) (end 199.6186 100.6602) (width 0.8) (layer B.Cu) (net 1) (status 10))
 (segment (start 201.93 111.125) (end 201.93 100.6856) (width 0.8) (layer B.Cu) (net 1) (status 10))
 (segment (start 199.644 100.6856) (end 199.517 100.5586) (width 0.8) (layer B.Cu) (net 1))
 (segment (start 201.93 100.6856) (end 199.644 100.6856) (width 0.8) (layer B.Cu) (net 1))
 (segment (start 212.8012 89.1032) (end 212.8012 84.62601) (width 0.4) (layer F.Cu) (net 1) (status 10))
 (segment (start 212.8012 84.62601) (end 202.4888 84.62601) (width 0.4) (layer F.Cu) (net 1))
 (segment (start 202.438 84.67681) (end 202.438 86.233) (width 0.4) (layer F.Cu) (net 1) (status 20))
 (segment (start 202.4888 84.62601) (end 202.438 84.67681) (width 0.4) (layer F.Cu) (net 1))
 (segment (start 223.2152 89.1032) (end 223.2152 84.62601) (width 0.4) (layer F.Cu) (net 1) (status 10))
 (segment (start 223.2152 84.62601) (end 212.8012 84.62601) (width 0.4) (layer F.Cu) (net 1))
 (segment (start 196.1134 99.0264) (end 196.1456 99.0586) (width 0.8) (layer B.Cu) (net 2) (status 30))
 (segment (start 196.1134 95.5802) (end 196.1134 99.0264) (width 0.8) (layer B.Cu) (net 2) (status 30))
 (segment (start 199.6043 95.5802) (end 199.6186 95.5659) (width 0.8) (layer B.Cu) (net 2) (status 30))
 (segment (start 196.1134 95.5802) (end 199.6043 95.5802) (width 0.8) (layer B.Cu) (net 2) (status 30))
 (segment (start 217.8812 89.1032) (end 217.8812 84.62601) (width 0.4) (layer B.Cu) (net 2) (status 10))
 (segment (start 228.2952 84.62601) (end 228.2952 89.1032) (width 0.4) (layer B.Cu) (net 2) (status 20))
 (segment (start 218.23001 84.62601) (end 228.2952 84.62601) (width 0.4) (layer B.Cu) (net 2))
 (segment (start 207.518 84.6328) (end 207.52479 84.62601) (width 0.4) (layer B.Cu) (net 2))
 (segment (start 207.518 86.233) (end 207.518 84.6328) (width 0.4) (layer B.Cu) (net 2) (status 10))
 (segment (start 217.8812 84.62601) (end 218.23001 84.62601) (width 0.4) (layer B.Cu) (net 2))
 (segment (start 196.088 84.62601) (end 209.08601 84.62601) (width 0.4) (layer B.Cu) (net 2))
 (segment (start 196.088 94.5798) (end 196.088 84.62601) (width 0.4) (layer B.Cu) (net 2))
 (segment (start 196.1134 95.5802) (end 196.1134 94.6052) (width 0.4) (layer B.Cu) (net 2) (status 10))
 (segment (start 209.08601 84.62601) (end 218.23001 84.62601) (width 0.4) (layer B.Cu) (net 2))
 (segment (start 196.1134 94.6052) (end 196.088 94.5798) (width 0.4) (layer B.Cu) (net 2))
 (segment (start 207.52479 84.62601) (end 209.08601 84.62601) (width 0.4) (layer B.Cu) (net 2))
 (segment (start 207.6069 86.3219) (end 207.518 86.233) (width 0.4) (layer B.Cu) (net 2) (status 30))
 (segment (start 207.6069 91.5273) (end 207.6069 86.3219) (width 0.4) (layer B.Cu) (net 2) (status 30))
 (segment (start 212.190999 97.477799) (end 212.1916 97.477198) (width 0.4) (layer B.Cu) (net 2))
 (segment (start 212.191 98.6028) (end 212.190999 97.477799) (width 0.4) (layer B.Cu) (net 2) (status 10))
 (segment (start 212.1916 97.477198) (end 212.1916 96.4184) (width 0.4) (layer B.Cu) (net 2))
 (segment (start 200.4711 96.4184) (end 199.6186 95.5659) (width 0.4) (layer B.Cu) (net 2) (status 20))
 (segment (start 212.1916 96.4184) (end 200.4711 96.4184) (width 0.4) (layer B.Cu) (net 2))
 (segment (start 196.1456 105.6708) (end 196.1642 105.6894) (width 0.8) (layer B.Cu) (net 3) (status 30))
 (segment (start 196.1456 102.0586) (end 196.1456 105.6708) (width 0.8) (layer B.Cu) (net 3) (status 30))
 (segment (start 199.5535 105.6894) (end 199.5678 105.7037) (width 0.8) (layer B.Cu) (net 3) (status 30))
 (segment (start 196.1642 105.6894) (end 199.5535 105.6894) (width 0.8) (layer B.Cu) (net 3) (status 30))
 (segment (start 192.922 108.4744) (end 192.922 110.744) (width 0.8) (layer B.Cu) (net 3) (status 20))
 (segment (start 193.2432 108.1532) (end 192.922 108.4744) (width 0.8) (layer B.Cu) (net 3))
 (segment (start 196.1388 106.6898) (end 196.1388 108.1532) (width 0.8) (layer B.Cu) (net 3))
 (segment (start 196.1642 105.6894) (end 196.1642 106.6644) (width 0.8) (layer B.Cu) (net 3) (status 10))
 (segment (start 196.1388 108.1532) (end 193.2432 108.1532) (width 0.8) (layer B.Cu) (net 3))
 (segment (start 196.1642 106.6644) (end 196.1388 106.6898) (width 0.8) (layer B.Cu) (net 3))
 (segment (start 207.6016 94.497) (end 207.6069 94.5023) (width 0.4) (layer B.Cu) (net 6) (status 30))
 (segment (start 204.2541 94.497) (end 207.6016 94.497) (width 0.4) (layer B.Cu) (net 6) (status 30))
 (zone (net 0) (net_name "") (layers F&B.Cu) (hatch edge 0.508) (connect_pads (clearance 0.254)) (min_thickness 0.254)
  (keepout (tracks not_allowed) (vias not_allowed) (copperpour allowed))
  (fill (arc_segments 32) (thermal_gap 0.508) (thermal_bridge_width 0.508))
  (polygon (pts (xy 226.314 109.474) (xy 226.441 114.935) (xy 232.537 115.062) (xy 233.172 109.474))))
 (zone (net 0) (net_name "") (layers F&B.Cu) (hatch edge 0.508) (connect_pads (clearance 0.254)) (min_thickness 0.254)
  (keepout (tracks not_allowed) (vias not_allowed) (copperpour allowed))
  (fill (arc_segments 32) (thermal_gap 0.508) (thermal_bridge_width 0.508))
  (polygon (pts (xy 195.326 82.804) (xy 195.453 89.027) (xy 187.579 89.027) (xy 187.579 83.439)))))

